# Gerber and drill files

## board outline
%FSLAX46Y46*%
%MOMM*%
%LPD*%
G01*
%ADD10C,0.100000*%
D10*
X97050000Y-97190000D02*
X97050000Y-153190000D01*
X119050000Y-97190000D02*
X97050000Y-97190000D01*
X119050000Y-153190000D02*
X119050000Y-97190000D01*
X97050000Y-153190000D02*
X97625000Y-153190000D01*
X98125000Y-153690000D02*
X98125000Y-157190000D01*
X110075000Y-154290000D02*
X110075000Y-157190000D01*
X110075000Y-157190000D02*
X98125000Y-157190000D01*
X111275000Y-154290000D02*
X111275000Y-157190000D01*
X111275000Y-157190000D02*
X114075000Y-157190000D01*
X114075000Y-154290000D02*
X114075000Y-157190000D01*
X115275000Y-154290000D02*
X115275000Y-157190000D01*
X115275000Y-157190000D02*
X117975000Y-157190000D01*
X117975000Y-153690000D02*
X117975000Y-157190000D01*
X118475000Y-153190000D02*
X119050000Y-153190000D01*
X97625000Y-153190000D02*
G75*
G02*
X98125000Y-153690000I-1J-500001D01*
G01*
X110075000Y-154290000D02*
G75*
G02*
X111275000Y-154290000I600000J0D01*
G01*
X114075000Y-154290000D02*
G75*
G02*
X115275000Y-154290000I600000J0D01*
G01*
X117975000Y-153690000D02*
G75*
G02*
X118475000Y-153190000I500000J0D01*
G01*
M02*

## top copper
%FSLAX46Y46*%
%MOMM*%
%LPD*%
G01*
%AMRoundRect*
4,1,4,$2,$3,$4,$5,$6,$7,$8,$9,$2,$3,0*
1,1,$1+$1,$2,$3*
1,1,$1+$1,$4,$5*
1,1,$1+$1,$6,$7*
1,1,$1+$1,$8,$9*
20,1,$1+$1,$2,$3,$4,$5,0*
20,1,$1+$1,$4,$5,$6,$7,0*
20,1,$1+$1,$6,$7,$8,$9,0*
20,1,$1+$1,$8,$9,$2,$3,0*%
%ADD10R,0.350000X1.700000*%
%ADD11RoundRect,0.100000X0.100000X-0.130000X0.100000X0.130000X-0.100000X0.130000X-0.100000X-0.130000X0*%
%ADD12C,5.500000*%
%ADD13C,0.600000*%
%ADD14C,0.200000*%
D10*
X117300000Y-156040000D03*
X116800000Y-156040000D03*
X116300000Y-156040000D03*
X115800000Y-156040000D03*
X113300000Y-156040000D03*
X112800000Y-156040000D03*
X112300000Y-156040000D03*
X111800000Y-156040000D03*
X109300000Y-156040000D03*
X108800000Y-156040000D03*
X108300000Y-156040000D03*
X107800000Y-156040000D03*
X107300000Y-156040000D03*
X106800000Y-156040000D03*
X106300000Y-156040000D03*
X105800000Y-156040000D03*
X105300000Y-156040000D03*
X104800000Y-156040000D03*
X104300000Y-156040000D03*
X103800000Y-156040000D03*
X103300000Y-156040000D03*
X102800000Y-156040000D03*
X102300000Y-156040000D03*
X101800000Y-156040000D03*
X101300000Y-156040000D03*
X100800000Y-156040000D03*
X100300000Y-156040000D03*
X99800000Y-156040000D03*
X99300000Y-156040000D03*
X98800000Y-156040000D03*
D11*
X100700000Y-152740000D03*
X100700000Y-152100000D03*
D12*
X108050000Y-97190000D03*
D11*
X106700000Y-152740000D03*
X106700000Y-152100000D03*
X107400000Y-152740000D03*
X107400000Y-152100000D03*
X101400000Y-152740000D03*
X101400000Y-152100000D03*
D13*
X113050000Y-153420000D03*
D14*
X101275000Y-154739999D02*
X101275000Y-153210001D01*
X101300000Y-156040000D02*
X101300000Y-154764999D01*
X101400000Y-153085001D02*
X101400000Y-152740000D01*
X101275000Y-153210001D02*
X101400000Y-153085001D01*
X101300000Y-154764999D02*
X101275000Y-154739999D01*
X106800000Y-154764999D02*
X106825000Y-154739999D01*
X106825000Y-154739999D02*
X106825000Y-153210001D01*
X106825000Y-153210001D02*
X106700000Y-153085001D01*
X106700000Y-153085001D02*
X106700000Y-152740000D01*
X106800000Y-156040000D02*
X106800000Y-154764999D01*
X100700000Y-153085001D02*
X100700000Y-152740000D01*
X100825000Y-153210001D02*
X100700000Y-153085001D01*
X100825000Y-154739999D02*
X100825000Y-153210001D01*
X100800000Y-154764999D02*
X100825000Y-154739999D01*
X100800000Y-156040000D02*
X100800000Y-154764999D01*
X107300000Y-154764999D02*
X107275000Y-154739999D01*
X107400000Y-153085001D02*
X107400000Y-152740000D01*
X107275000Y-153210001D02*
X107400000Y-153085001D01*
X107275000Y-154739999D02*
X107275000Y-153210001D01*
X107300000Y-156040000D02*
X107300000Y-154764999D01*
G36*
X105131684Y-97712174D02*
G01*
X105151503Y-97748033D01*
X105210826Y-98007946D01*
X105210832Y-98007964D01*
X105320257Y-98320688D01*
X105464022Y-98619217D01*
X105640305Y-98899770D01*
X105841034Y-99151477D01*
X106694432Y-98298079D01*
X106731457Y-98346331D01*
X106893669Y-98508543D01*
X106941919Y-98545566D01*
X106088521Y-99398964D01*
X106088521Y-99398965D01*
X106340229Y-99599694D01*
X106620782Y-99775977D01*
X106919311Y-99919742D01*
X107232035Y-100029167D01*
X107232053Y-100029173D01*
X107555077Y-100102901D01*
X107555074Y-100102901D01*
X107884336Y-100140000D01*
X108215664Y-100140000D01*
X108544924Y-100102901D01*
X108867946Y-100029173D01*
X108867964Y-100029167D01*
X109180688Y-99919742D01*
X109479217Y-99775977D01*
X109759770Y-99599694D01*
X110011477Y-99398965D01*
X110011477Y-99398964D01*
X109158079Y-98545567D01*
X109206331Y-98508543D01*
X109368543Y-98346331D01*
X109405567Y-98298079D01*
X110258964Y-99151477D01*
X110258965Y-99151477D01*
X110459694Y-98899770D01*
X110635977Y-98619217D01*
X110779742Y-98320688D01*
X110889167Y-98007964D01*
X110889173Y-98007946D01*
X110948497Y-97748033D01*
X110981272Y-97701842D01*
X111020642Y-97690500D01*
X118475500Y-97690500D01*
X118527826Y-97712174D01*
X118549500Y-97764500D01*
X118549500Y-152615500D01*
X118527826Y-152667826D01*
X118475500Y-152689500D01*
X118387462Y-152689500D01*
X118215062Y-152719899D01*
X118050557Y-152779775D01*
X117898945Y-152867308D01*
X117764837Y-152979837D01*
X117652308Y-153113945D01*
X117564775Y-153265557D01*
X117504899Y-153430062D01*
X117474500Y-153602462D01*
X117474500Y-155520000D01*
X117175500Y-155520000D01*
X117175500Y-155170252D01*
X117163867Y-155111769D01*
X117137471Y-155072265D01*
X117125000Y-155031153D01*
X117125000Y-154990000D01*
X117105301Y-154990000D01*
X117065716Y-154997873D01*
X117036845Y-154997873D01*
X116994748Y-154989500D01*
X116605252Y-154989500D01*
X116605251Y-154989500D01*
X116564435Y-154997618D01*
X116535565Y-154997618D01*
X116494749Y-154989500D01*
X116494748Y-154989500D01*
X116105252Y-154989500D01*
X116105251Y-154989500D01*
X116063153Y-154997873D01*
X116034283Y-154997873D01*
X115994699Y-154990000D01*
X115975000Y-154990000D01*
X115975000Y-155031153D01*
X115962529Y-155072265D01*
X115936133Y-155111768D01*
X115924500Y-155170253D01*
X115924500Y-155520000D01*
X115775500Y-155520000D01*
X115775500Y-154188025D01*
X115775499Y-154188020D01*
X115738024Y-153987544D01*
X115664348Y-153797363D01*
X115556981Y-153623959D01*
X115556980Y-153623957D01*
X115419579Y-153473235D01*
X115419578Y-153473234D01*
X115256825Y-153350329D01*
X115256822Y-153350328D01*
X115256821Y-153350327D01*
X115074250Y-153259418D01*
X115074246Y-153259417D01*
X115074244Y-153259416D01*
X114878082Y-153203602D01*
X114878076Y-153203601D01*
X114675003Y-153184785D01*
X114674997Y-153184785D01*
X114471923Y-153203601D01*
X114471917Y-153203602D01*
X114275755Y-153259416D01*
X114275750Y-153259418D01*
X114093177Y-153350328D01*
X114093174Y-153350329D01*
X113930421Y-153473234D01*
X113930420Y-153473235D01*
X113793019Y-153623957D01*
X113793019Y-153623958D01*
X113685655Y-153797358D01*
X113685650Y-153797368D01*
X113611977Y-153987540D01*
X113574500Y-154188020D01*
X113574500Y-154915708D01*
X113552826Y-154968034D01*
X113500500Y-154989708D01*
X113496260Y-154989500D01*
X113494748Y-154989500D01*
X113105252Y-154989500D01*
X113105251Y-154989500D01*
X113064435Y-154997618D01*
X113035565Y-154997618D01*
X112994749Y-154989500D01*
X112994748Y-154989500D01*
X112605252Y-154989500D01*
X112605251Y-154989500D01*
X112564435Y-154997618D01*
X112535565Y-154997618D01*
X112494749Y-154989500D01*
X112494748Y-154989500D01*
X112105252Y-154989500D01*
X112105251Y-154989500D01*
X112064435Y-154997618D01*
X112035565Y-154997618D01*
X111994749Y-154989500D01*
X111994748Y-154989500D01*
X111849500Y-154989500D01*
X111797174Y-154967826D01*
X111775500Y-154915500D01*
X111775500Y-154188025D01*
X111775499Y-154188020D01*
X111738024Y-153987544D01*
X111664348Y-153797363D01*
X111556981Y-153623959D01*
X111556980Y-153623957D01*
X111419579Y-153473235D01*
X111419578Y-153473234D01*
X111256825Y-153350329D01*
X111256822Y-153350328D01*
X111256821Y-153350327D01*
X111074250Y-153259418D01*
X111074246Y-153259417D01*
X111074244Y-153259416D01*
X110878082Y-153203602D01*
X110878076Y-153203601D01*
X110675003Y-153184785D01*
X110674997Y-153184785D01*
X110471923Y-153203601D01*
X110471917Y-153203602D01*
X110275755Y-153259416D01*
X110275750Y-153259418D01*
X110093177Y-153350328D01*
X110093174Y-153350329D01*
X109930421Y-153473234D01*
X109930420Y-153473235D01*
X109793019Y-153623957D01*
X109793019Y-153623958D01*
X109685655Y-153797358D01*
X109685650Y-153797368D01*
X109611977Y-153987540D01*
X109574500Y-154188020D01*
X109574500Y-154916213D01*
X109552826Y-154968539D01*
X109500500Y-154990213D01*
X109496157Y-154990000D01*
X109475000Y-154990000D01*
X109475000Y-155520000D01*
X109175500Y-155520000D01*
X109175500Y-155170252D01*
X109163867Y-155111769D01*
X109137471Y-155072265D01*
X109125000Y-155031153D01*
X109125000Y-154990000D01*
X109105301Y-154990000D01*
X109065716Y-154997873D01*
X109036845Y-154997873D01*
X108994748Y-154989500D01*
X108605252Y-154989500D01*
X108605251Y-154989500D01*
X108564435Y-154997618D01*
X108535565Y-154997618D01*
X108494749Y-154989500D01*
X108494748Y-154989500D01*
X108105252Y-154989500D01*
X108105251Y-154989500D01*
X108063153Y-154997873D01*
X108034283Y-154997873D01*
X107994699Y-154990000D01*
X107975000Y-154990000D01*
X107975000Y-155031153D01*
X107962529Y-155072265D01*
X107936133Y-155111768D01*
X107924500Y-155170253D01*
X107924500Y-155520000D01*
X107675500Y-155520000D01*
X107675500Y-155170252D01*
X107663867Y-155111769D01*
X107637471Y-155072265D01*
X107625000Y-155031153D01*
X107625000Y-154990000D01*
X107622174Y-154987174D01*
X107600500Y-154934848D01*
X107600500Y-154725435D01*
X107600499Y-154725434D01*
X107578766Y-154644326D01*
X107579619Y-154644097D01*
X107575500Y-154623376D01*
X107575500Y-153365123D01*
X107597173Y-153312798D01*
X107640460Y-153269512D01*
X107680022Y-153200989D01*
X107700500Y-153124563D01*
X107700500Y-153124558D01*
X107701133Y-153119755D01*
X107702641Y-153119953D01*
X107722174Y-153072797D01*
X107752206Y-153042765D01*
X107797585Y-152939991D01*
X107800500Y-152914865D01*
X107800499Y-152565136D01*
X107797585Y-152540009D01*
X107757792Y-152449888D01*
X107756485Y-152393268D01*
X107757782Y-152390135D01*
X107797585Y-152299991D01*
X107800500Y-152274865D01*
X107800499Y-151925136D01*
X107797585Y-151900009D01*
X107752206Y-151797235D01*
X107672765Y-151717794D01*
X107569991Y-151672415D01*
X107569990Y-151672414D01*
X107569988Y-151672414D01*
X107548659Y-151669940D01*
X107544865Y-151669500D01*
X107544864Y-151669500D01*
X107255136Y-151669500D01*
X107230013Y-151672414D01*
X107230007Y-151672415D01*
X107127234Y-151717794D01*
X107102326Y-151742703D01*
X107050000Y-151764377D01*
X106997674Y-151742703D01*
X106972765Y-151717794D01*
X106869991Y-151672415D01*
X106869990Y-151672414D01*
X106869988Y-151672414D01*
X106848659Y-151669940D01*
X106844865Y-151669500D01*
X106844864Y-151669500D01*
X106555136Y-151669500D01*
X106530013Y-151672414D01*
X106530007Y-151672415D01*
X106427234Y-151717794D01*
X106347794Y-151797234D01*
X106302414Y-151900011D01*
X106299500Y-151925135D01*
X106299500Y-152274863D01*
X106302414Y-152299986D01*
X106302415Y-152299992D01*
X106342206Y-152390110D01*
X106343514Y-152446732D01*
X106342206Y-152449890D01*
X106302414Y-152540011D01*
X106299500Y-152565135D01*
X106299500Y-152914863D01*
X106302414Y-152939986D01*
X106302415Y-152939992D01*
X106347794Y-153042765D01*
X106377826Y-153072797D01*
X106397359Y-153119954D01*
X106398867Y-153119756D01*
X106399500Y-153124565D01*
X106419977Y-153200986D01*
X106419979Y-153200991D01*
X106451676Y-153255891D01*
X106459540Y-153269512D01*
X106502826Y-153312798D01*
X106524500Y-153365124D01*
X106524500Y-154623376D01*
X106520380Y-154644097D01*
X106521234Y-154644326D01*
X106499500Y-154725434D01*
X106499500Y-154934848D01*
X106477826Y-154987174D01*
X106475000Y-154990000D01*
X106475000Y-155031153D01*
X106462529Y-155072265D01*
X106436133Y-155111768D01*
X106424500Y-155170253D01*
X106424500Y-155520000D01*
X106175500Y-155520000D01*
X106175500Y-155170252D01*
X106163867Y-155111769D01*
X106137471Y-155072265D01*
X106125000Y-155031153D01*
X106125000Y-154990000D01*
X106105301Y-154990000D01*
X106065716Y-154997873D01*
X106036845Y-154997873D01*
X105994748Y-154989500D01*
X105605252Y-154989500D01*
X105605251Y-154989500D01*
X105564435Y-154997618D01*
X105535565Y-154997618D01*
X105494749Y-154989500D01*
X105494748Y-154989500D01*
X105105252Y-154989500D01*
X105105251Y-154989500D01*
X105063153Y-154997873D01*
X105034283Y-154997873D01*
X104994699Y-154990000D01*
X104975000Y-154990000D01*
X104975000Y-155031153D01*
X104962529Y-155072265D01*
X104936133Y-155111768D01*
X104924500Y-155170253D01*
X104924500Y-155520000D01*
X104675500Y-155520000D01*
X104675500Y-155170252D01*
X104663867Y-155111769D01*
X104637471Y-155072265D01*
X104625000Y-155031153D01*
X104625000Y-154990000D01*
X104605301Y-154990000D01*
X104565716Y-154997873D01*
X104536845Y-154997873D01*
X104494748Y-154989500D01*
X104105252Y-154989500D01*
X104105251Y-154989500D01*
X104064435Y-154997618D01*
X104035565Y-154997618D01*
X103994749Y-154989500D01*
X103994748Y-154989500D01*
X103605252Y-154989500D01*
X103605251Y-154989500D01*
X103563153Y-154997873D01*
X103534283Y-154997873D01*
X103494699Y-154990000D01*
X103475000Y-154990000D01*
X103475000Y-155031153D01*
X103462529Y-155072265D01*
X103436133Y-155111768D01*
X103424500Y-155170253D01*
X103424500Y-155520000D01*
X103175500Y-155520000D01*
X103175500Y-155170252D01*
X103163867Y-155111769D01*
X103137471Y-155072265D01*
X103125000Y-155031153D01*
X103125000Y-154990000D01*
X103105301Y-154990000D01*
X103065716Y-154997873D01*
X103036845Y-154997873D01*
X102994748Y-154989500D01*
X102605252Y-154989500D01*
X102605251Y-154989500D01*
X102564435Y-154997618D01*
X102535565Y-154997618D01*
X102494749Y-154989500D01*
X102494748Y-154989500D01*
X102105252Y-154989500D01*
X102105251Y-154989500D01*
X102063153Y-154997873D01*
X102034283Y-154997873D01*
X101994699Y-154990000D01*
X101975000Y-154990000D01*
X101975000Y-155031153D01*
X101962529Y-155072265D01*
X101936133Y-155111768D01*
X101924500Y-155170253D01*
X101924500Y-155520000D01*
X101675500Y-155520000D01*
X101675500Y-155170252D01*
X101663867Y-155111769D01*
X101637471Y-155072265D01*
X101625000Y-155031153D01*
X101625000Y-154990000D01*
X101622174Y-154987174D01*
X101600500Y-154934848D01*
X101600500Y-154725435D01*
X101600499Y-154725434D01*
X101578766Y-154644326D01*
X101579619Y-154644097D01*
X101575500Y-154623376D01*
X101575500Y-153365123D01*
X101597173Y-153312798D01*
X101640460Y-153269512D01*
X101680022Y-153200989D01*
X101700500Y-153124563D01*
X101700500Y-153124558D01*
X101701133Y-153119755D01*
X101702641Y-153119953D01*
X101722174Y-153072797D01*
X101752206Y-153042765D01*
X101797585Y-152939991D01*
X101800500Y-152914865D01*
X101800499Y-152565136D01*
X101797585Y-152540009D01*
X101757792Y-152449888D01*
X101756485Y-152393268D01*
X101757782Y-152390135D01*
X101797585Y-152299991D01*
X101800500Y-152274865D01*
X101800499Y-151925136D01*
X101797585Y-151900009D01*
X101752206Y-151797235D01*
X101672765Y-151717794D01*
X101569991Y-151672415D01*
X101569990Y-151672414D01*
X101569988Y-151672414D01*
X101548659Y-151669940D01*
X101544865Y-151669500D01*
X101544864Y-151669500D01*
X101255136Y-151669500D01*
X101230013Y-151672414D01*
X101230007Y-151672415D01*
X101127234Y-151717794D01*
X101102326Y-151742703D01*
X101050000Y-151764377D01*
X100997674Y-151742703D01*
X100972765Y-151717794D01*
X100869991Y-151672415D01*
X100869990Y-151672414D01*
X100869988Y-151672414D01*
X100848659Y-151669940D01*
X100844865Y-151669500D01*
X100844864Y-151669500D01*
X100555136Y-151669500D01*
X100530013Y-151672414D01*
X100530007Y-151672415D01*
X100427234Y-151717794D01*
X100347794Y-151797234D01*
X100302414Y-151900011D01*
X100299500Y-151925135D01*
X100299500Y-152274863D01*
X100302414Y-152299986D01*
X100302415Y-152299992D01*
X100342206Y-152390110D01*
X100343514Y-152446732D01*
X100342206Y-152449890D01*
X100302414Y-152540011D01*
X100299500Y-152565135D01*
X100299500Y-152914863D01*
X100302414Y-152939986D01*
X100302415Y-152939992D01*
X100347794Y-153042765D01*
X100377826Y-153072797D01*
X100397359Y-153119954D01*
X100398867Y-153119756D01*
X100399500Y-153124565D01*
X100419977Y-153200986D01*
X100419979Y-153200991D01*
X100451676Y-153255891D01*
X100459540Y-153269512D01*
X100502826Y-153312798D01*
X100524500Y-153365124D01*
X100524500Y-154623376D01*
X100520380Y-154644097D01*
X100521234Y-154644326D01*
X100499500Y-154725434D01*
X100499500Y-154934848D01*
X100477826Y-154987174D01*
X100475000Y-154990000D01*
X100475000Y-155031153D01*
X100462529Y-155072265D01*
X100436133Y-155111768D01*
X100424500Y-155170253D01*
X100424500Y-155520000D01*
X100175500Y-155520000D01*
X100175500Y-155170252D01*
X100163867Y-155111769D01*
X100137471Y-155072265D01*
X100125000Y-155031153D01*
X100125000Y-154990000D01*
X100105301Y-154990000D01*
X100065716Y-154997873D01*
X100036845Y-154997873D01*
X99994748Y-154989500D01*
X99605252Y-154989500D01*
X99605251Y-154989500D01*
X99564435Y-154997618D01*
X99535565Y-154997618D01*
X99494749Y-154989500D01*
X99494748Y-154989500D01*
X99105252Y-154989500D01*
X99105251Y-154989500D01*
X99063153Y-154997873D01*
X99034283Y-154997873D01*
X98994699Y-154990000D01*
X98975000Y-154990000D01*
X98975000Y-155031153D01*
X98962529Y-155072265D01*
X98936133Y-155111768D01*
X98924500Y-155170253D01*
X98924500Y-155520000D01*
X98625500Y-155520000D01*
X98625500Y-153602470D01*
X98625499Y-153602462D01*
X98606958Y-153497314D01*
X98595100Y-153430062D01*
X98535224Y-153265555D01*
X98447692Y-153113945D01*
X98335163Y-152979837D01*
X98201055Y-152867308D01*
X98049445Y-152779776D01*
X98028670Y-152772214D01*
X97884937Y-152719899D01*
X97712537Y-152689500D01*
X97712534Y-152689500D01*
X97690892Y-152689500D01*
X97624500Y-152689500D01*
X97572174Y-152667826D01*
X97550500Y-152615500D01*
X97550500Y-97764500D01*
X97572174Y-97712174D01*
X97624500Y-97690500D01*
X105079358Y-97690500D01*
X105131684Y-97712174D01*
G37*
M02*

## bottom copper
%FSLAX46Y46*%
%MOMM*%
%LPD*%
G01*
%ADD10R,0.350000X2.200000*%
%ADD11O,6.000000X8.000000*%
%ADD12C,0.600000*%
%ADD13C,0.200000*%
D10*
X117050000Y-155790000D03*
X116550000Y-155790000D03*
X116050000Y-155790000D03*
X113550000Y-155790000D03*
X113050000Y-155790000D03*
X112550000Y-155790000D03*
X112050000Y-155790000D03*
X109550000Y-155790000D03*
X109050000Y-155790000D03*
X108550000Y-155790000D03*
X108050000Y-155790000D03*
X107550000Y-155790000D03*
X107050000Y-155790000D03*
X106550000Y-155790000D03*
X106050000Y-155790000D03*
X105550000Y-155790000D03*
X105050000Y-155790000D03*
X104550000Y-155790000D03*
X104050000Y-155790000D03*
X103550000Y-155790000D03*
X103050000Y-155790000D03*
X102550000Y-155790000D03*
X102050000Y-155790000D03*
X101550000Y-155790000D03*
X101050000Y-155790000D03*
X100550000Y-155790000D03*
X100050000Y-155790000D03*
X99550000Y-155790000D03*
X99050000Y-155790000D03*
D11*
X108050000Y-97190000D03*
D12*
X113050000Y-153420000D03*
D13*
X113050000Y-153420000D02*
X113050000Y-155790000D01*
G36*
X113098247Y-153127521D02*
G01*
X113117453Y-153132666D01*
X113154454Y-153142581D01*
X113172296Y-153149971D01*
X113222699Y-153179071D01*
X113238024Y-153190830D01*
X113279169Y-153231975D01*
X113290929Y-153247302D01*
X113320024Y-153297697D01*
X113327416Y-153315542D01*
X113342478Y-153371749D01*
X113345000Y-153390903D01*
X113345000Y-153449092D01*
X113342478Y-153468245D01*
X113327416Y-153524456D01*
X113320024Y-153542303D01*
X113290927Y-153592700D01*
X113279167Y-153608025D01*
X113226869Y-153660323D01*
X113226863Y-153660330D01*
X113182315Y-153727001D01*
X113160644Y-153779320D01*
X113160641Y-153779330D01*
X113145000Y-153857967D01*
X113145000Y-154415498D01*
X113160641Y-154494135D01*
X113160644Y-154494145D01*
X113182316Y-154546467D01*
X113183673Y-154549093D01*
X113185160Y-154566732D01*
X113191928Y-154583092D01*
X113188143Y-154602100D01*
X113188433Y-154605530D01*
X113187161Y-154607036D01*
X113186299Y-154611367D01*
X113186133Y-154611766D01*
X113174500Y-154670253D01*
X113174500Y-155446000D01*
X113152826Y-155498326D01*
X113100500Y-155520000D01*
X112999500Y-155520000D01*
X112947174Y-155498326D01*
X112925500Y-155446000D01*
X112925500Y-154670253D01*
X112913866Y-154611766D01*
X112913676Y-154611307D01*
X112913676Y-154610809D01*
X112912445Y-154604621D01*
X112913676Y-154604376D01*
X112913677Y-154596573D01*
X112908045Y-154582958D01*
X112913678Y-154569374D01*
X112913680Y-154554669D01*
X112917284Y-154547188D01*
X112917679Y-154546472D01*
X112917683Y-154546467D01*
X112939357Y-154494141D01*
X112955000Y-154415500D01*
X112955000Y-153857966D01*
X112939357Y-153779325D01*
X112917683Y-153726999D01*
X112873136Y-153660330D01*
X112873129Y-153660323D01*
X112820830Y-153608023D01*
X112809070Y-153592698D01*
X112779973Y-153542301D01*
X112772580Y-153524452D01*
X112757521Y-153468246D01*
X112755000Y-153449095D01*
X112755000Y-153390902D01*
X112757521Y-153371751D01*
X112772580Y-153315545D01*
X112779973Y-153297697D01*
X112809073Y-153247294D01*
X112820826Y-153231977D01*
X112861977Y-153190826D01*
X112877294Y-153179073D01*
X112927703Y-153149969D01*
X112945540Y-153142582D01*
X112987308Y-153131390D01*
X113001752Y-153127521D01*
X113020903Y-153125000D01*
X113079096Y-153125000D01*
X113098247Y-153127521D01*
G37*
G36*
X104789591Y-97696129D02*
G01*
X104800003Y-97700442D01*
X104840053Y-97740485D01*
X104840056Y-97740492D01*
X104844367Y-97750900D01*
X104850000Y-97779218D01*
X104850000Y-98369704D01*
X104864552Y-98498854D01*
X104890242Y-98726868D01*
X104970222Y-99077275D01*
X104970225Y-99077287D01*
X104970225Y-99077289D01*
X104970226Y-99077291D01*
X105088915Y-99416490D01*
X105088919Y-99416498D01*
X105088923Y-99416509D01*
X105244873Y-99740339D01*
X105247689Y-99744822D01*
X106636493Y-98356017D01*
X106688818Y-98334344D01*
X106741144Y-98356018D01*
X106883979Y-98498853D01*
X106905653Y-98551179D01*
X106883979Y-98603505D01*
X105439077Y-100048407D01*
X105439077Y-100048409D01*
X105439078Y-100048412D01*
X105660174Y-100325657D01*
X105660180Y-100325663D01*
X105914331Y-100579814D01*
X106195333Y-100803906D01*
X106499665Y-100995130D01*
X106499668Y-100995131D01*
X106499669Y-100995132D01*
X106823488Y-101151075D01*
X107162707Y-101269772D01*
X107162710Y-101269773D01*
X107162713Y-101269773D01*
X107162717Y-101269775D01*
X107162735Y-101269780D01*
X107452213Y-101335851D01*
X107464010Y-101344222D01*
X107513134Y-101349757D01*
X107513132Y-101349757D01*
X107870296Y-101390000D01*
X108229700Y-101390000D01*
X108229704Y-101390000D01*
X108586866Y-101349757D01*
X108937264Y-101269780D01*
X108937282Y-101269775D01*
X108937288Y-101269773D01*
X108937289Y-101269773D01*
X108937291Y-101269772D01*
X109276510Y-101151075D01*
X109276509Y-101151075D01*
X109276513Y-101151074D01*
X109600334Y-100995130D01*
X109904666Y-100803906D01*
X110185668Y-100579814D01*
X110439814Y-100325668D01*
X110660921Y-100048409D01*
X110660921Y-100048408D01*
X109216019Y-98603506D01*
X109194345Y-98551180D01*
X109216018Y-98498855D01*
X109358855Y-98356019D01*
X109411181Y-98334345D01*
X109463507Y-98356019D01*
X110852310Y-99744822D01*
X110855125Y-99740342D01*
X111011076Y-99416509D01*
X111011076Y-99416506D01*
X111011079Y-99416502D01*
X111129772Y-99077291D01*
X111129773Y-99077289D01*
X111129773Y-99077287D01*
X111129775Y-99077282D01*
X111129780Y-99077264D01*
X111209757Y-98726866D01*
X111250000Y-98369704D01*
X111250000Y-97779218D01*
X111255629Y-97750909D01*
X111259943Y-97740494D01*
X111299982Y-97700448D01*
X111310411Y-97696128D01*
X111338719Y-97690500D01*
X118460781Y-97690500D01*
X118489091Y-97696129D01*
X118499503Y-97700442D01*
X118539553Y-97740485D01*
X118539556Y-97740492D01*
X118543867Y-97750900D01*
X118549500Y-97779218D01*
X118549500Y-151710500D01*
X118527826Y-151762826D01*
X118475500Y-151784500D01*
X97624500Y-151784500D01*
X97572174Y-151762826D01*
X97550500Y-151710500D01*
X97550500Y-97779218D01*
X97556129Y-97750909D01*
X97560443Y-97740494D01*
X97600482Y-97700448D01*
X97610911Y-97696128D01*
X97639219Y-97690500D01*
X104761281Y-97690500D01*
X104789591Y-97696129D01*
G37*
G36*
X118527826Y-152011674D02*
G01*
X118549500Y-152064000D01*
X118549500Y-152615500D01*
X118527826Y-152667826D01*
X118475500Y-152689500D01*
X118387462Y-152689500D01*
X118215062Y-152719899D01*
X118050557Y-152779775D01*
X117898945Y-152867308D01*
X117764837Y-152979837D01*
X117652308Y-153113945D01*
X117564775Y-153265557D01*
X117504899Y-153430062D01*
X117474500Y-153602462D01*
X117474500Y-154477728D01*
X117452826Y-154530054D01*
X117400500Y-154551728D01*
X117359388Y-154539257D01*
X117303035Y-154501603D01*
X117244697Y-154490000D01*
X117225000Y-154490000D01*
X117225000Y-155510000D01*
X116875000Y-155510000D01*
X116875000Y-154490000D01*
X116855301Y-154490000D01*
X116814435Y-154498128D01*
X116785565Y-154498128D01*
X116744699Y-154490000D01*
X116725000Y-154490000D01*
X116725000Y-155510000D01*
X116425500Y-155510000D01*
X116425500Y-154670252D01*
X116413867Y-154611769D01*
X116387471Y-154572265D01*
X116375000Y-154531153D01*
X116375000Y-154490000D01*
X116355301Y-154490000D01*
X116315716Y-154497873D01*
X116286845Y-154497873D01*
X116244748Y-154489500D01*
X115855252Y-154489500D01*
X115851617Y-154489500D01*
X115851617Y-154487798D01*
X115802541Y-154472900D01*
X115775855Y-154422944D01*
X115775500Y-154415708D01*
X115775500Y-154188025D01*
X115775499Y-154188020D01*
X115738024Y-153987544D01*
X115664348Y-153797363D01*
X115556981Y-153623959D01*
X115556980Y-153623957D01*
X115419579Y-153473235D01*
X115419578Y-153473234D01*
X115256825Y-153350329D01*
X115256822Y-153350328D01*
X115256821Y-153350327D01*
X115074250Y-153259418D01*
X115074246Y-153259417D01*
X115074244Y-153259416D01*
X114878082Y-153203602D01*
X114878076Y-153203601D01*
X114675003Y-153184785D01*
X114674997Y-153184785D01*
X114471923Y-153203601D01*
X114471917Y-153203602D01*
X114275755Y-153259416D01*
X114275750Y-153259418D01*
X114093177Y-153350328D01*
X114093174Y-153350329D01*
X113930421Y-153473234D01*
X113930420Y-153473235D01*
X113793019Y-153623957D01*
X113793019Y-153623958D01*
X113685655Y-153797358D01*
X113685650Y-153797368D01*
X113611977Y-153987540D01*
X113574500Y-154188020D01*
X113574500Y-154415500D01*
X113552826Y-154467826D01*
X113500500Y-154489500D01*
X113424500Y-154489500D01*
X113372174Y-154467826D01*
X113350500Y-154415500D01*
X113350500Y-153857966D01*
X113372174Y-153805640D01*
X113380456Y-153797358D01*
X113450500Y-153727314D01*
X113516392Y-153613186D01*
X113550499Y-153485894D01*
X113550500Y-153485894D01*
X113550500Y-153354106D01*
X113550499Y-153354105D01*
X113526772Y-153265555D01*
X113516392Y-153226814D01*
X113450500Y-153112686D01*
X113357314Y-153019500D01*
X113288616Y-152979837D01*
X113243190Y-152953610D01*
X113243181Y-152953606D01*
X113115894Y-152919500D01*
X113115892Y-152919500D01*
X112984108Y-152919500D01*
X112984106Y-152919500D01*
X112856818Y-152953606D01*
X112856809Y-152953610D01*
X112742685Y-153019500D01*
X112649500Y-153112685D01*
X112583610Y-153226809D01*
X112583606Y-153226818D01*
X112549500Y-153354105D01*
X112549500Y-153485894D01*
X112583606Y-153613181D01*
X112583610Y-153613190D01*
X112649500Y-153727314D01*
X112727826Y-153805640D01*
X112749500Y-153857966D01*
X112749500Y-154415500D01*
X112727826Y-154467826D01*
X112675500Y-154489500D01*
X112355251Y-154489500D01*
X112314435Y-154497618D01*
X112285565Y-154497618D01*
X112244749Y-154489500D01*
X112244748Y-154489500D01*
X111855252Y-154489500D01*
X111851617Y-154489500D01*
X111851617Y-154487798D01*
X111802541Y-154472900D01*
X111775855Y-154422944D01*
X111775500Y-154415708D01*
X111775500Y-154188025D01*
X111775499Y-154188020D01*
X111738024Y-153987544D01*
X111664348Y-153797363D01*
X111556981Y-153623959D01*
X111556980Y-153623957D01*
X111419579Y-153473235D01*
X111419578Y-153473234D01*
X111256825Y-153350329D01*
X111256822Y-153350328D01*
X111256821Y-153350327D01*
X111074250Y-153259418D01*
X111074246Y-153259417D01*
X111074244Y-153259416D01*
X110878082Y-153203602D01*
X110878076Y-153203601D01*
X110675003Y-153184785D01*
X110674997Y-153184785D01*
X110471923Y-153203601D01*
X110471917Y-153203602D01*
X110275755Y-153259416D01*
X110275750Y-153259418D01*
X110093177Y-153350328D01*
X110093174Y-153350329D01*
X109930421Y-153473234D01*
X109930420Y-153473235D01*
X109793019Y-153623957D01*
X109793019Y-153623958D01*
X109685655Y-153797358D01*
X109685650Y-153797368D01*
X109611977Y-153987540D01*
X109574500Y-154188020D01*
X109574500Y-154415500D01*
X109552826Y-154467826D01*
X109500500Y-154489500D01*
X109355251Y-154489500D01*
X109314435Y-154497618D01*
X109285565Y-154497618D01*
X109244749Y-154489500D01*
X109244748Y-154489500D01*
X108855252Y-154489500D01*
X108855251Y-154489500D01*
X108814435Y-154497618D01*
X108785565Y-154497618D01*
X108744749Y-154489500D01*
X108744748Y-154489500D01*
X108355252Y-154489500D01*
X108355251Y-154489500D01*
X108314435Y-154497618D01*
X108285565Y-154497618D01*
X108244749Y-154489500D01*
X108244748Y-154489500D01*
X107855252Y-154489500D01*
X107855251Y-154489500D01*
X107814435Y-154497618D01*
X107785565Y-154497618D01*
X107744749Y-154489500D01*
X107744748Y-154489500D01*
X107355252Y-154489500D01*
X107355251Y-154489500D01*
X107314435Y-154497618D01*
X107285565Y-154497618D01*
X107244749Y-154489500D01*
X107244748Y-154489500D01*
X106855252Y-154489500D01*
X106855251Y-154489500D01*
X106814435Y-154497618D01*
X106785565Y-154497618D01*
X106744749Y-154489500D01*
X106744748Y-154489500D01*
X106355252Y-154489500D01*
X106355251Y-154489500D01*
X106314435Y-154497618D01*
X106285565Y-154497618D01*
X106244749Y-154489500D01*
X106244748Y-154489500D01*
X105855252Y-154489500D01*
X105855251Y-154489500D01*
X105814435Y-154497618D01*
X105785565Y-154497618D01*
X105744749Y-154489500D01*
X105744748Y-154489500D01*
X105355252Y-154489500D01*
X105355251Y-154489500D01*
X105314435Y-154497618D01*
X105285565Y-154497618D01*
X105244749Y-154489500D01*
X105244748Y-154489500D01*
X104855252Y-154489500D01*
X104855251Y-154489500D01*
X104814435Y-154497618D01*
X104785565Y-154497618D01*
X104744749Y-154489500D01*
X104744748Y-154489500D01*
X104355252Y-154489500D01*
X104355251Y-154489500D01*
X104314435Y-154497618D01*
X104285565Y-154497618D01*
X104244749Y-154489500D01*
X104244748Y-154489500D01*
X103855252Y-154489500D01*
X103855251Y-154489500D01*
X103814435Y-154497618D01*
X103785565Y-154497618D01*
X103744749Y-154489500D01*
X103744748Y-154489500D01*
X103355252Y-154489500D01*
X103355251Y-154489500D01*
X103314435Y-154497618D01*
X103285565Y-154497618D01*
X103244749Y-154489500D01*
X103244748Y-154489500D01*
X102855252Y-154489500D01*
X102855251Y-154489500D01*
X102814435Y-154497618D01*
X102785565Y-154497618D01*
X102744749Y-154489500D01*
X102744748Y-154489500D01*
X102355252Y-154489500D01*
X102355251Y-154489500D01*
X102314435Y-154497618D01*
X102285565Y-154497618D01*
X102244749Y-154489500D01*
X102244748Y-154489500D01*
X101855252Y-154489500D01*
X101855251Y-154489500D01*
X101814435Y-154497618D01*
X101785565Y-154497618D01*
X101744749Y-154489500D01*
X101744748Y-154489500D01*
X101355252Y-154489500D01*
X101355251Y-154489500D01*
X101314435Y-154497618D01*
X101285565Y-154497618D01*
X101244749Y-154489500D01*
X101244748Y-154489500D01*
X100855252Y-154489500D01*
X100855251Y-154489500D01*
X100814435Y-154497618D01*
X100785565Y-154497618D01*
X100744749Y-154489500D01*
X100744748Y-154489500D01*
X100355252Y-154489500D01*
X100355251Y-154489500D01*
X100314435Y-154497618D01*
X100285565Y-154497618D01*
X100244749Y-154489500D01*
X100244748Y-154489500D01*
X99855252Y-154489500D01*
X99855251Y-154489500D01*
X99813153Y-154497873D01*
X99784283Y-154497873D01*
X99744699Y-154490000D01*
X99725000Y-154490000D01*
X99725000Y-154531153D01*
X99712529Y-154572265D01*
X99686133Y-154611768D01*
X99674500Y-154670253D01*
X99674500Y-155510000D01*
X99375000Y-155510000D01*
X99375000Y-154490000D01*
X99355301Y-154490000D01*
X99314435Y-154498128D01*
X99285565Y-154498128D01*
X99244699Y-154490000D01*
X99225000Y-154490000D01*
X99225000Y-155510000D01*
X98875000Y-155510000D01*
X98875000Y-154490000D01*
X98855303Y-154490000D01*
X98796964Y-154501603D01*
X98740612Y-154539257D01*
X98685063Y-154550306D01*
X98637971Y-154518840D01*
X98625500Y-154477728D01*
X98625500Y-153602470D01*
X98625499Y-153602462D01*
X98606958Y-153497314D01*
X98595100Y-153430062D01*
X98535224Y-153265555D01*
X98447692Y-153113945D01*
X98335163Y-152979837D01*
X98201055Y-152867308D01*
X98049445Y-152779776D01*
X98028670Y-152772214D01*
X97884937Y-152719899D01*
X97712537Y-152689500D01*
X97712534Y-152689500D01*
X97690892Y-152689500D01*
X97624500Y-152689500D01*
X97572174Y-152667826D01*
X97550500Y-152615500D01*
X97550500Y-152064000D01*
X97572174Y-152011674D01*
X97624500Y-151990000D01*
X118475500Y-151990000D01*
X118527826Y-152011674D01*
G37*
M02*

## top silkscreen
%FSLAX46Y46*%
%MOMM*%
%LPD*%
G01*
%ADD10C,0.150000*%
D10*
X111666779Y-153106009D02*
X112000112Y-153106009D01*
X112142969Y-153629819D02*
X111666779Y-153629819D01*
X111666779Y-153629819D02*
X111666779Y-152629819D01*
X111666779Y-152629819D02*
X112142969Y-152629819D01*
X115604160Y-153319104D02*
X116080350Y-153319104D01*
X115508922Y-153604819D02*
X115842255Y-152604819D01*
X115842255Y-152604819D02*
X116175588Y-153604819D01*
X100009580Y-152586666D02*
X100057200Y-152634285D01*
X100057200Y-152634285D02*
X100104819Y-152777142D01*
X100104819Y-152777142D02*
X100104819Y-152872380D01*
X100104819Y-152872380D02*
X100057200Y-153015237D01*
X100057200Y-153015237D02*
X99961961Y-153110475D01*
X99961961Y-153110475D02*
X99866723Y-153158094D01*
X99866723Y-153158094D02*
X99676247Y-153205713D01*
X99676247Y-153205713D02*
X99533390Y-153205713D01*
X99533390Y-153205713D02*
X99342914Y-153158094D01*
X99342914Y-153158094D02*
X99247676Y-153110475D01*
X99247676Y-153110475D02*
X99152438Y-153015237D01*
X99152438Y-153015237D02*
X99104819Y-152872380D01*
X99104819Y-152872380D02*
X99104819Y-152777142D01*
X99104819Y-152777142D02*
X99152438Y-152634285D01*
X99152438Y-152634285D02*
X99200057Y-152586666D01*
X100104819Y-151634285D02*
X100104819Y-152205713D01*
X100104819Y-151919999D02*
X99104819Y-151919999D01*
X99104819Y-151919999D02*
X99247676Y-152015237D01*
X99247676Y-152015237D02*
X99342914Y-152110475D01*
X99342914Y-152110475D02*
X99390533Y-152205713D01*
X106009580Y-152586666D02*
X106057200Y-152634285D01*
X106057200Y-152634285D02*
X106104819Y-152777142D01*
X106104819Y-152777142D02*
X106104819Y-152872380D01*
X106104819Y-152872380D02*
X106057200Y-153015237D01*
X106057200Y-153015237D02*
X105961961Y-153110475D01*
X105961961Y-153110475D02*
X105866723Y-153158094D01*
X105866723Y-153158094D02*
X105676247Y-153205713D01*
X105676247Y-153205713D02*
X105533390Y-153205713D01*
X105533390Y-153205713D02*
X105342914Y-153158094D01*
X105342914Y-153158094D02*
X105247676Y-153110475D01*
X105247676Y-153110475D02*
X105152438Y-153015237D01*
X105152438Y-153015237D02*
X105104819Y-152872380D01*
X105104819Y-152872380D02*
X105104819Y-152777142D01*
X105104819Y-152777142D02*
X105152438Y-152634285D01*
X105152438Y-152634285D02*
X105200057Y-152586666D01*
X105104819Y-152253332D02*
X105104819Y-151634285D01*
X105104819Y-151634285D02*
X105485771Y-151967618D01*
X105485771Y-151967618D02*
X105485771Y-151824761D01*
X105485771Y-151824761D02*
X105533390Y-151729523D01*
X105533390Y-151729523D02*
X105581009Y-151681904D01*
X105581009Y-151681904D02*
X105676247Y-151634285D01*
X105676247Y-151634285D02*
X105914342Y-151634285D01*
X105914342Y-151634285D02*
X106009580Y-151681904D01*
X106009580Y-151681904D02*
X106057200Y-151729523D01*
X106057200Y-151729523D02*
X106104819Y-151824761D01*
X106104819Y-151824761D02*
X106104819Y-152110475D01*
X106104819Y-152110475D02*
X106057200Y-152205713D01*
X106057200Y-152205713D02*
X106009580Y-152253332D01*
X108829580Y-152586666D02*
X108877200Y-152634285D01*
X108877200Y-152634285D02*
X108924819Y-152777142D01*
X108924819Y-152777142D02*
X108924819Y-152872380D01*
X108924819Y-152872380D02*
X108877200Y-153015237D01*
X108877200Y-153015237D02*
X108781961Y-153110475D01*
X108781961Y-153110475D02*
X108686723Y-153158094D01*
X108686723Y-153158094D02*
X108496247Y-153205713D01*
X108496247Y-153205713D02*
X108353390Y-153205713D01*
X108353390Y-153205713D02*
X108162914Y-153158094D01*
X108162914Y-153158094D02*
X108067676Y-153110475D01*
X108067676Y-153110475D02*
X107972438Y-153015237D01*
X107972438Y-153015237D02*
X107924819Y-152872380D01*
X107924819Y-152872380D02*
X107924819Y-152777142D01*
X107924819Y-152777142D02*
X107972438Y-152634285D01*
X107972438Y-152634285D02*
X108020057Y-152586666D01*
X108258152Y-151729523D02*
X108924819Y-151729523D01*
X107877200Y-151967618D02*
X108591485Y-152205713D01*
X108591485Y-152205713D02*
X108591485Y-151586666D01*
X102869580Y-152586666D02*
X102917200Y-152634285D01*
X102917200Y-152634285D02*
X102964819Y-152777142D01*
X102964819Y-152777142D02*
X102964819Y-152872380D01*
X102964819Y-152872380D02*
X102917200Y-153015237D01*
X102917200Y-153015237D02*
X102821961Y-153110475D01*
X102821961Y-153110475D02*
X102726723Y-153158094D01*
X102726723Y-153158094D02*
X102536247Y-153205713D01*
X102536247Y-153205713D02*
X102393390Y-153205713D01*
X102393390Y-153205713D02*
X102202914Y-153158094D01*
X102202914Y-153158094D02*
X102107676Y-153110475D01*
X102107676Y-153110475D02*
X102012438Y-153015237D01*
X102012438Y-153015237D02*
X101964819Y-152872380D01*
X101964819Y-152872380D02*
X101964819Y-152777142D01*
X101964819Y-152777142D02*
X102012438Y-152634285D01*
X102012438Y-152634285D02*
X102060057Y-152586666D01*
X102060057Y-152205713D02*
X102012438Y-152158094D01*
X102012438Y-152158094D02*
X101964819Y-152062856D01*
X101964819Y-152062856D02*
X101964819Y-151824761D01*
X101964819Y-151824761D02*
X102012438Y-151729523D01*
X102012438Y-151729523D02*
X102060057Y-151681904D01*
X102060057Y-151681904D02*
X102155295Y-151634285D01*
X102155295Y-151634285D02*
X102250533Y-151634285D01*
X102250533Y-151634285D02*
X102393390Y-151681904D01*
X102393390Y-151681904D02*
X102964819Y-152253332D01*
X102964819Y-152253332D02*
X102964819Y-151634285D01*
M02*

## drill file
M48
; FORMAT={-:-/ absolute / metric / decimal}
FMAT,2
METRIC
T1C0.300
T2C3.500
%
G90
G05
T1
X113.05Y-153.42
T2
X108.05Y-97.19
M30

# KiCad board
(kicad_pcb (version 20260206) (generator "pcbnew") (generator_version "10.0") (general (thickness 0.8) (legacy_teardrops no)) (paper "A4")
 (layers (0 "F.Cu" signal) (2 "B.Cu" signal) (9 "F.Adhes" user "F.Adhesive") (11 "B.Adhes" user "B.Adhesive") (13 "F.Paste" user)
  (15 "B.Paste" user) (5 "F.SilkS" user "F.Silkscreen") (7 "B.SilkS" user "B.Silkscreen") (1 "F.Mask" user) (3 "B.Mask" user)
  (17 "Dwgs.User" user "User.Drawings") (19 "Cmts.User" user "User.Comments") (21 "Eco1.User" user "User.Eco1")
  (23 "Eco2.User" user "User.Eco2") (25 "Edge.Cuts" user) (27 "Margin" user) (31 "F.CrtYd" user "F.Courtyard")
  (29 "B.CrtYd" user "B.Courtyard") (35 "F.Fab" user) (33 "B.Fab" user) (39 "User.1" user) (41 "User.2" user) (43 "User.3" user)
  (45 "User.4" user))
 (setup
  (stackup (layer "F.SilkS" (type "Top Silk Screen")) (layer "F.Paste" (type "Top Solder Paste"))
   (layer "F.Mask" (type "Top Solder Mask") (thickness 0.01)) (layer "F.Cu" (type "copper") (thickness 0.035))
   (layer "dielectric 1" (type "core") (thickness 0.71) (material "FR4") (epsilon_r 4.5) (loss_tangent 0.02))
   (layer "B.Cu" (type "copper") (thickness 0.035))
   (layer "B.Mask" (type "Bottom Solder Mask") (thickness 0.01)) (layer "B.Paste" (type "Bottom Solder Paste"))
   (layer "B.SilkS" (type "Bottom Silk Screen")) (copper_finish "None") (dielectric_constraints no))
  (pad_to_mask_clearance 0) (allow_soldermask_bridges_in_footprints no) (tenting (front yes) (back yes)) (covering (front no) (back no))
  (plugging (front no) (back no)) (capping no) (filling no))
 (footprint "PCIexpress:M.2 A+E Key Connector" (layer "F.Cu") (at 108.05 156.08)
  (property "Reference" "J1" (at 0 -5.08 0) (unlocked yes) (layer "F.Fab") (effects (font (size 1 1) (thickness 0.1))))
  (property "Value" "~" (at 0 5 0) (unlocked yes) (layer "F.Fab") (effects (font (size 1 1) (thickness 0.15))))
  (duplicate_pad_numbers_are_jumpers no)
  (fp_line (start -11 -2.89) (end -10.425 -2.89) (stroke (width 0.1) (type default)) (layer "Edge.Cuts"))
  (fp_line (start -9.925 -2.39) (end -9.925 1.11) (stroke (width 0.1) (type default)) (layer "Edge.Cuts"))
  (fp_line (start 2.025 -1.79) (end 2.025 1.11) (stroke (width 0.1) (type default)) (layer "Edge.Cuts"))
  (fp_line (start 2.025 1.11) (end -9.925 1.11) (stroke (width 0.1) (type default)) (layer "Edge.Cuts"))
  (fp_line (start 3.225 -1.79) (end 3.225 1.11) (stroke (width 0.1) (type default)) (layer "Edge.Cuts"))
  (fp_line (start 3.225 1.11) (end 6.025 1.11) (stroke (width 0.1) (type default)) (layer "Edge.Cuts"))
  (fp_line (start 6.025 -1.79) (end 6.025 1.11) (stroke (width 0.1) (type default)) (layer "Edge.Cuts"))
  (fp_line (start 7.225 -1.79) (end 7.225 1.11) (stroke (width 0.1) (type default)) (layer "Edge.Cuts"))
  (fp_line (start 7.225 1.11) (end 9.925 1.11) (stroke (width 0.1) (type default)) (layer "Edge.Cuts"))
  (fp_line (start 9.925 -2.39) (end 9.925 1.11) (stroke (width 0.1) (type default)) (layer "Edge.Cuts"))
  (fp_line (start 10.425 -2.89) (end 11 -2.89) (stroke (width 0.1) (type default)) (layer "Edge.Cuts"))
  (fp_arc (start -10.425 -2.89) (mid -10.071447 -2.743553) (end -9.925 -2.39) (stroke (width 0.1) (type default)) (layer "Edge.Cuts"))
  (fp_arc (start 2.025 -1.79) (mid 2.625 -2.39) (end 3.225 -1.79) (stroke (width 0.1) (type default)) (layer "Edge.Cuts"))
  (fp_arc (start 6.025 -1.79) (mid 6.625 -2.39) (end 7.225 -1.79) (stroke (width 0.1) (type default)) (layer "Edge.Cuts"))
  (fp_arc (start 9.925 -2.39) (mid 10.071447 -2.743553) (end 10.425 -2.89) (stroke (width 0.1) (type default)) (layer "Edge.Cuts"))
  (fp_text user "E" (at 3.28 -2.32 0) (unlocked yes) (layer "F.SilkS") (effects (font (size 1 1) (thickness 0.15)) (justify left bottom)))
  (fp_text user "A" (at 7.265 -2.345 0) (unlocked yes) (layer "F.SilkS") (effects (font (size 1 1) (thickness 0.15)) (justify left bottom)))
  (pad "1" smd rect (at 9.25 -0.04 180) (size 0.35 1.7) (layers "F.Cu") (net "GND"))
  (pad "2" smd rect (at 9 -0.29 180) (size 0.35 2.2) (layers "B.Cu") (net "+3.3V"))
  (pad "3" smd rect (at 8.75 -0.04 180) (size 0.35 1.7) (layers "F.Cu") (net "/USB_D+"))
  (pad "4" smd rect (at 8.5 -0.29 180) (size 0.35 2.2) (layers "B.Cu") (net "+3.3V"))
  (pad "5" smd rect (at 8.25 -0.04 180) (size 0.35 1.7) (layers "F.Cu") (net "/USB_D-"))
  (pad "6" smd rect (at 8 -0.29 180) (size 0.35 2.2) (layers "B.Cu") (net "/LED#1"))
  (pad "7" smd rect (at 7.75 -0.04 180) (size 0.35 1.7) (layers "F.Cu") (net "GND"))
  (pad "16" smd rect (at 5.5 -0.29 180) (size 0.35 2.2) (layers "B.Cu") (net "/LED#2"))
  (pad "17" smd rect (at 5.25 -0.04 180) (size 0.35 1.7) (layers "F.Cu") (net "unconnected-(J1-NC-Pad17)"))
  (pad "18" smd rect (at 5 -0.29 180) (size 0.35 2.2) (layers "B.Cu") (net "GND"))
  (pad "19" smd rect (at 4.75 -0.04 180) (size 0.35 1.7) (layers "F.Cu") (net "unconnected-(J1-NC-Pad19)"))
  (pad "20" smd rect (at 4.5 -0.29 180) (size 0.35 2.2) (layers "B.Cu") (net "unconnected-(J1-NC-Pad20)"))
  (pad "21" smd rect (at 4.25 -0.04 180) (size 0.35 1.7) (layers "F.Cu") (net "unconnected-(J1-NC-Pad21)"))
  (pad "22" smd rect (at 4 -0.29 180) (size 0.35 2.2) (layers "B.Cu") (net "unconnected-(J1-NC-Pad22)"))
  (pad "23" smd rect (at 3.75 -0.04 180) (size 0.35 1.7) (layers "F.Cu") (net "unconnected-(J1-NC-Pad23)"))
  (pad "32" smd rect (at 1.5 -0.29 180) (size 0.35 2.2) (layers "B.Cu") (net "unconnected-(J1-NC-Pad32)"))
  (pad "33" smd rect (at 1.25 -0.04 180) (size 0.35 1.7) (layers "F.Cu") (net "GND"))
  (pad "34" smd rect (at 1 -0.29 180) (size 0.35 2.2) (layers "B.Cu") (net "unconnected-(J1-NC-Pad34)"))
  (pad "35" smd rect (at 0.75 -0.04 180) (size 0.35 1.7) (layers "F.Cu") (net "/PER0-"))
  (pad "36" smd rect (at 0.5 -0.29 180) (size 0.35 2.2) (layers "B.Cu") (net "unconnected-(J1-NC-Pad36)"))
  (pad "37" smd rect (at 0.25 -0.04 180) (size 0.35 1.7) (layers "F.Cu") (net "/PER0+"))
  (pad "38" smd rect (at 0 -0.29 180) (size 0.35 2.2) (layers "B.Cu") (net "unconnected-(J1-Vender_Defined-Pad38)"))
  (pad "39" smd rect (at -0.25 -0.04 180) (size 0.35 1.7) (layers "F.Cu") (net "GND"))
  (pad "40" smd rect (at -0.5 -0.29 180) (size 0.35 2.2) (layers "B.Cu") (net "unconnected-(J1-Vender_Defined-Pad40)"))
  (pad "41" smd rect (at -0.75 -0.04 180) (size 0.35 1.7) (layers "F.Cu") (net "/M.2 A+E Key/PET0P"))
  (pad "42" smd rect (at -1 -0.29 180) (size 0.35 2.2) (layers "B.Cu") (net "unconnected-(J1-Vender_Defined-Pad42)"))
  (pad "43" smd rect (at -1.25 -0.04 180) (size 0.35 1.7) (layers "F.Cu") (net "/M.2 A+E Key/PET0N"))
  (pad "44" smd rect (at -1.5 -0.29 180) (size 0.35 2.2) (layers "B.Cu") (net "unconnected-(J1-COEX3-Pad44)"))
  (pad "45" smd rect (at -1.75 -0.04 180) (size 0.35 1.7) (layers "F.Cu") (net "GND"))
  (pad "46" smd rect (at -2 -0.29 180) (size 0.35 2.2) (layers "B.Cu") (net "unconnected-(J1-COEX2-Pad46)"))
  (pad "47" smd rect (at -2.25 -0.04 180) (size 0.35 1.7) (layers "F.Cu") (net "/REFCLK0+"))
  (pad "48" smd rect (at -2.5 -0.29 180) (size 0.35 2.2) (layers "B.Cu") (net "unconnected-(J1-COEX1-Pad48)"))
  (pad "49" smd rect (at -2.75 -0.04 180) (size 0.35 1.7) (layers "F.Cu") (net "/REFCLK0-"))
  (pad "50" smd rect (at -3 -0.29 180) (size 0.35 2.2) (layers "B.Cu") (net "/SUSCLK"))
  (pad "51" smd rect (at -3.25 -0.04 180) (size 0.35 1.7) (layers "F.Cu") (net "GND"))
  (pad "52" smd rect (at -3.5 -0.29 180) (size 0.35 2.2) (layers "B.Cu") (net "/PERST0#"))
  (pad "53" smd rect (at -3.75 -0.04 180) (size 0.35 1.7) (layers "F.Cu") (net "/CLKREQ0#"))
  (pad "54" smd rect (at -4 -0.29 180) (size 0.35 2.2) (layers "B.Cu") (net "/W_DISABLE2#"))
  (pad "55" smd rect (at -4.25 -0.04 180) (size 0.35 1.7) (layers "F.Cu") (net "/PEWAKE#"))
  (pad "56" smd rect (at -4.5 -0.29 180) (size 0.35 2.2) (layers "B.Cu") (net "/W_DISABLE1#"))
  (pad "57" smd rect (at -4.75 -0.04 180) (size 0.35 1.7) (layers "F.Cu") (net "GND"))
  (pad "58" smd rect (at -5 -0.29 180) (size 0.35 2.2) (layers "B.Cu") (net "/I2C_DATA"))
  (pad "59" smd rect (at -5.25 -0.04 180) (size 0.35 1.7) (layers "F.Cu") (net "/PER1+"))
  (pad "60" smd rect (at -5.5 -0.29 180) (size 0.35 2.2) (layers "B.Cu") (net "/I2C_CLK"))
  (pad "61" smd rect (at -5.75 -0.04 180) (size 0.35 1.7) (layers "F.Cu") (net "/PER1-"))
  (pad "62" smd rect (at -6 -0.29 180) (size 0.35 2.2) (layers "B.Cu") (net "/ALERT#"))
  (pad "63" smd rect (at -6.25 -0.04 180) (size 0.35 1.7) (layers "F.Cu") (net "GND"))
  (pad "64" smd rect (at -6.5 -0.29 180) (size 0.35 2.2) (layers "B.Cu") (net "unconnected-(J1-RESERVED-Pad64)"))
  (pad "65" smd rect (at -6.75 -0.04 180) (size 0.35 1.7) (layers "F.Cu") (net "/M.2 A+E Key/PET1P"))
  (pad "66" smd rect (at -7 -0.29 180) (size 0.35 2.2) (layers "B.Cu") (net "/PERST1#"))
  (pad "67" smd rect (at -7.25 -0.04 180) (size 0.35 1.7) (layers "F.Cu") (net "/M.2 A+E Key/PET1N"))
  (pad "68" smd rect (at -7.5 -0.29 180) (size 0.35 2.2) (layers "B.Cu") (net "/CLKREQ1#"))
  (pad "69" smd rect (at -7.75 -0.04 180) (size 0.35 1.7) (layers "F.Cu") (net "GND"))
  (pad "70" smd rect (at -8 -0.29 180) (size 0.35 2.2) (layers "B.Cu") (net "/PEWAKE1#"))
  (pad "71" smd rect (at -8.25 -0.04 180) (size 0.35 1.7) (layers "F.Cu") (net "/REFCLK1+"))
  (pad "72" smd rect (at -8.5 -0.29 180) (size 0.35 2.2) (layers "B.Cu") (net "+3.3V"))
  (pad "73" smd rect (at -8.75 -0.04 180) (size 0.35 1.7) (layers "F.Cu") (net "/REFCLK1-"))
  (pad "74" smd rect (at -9 -0.29 180) (size 0.35 2.2) (layers "B.Cu") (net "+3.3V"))
  (pad "75" smd rect (at -9.25 -0.04 180) (size 0.35 1.7) (layers "F.Cu") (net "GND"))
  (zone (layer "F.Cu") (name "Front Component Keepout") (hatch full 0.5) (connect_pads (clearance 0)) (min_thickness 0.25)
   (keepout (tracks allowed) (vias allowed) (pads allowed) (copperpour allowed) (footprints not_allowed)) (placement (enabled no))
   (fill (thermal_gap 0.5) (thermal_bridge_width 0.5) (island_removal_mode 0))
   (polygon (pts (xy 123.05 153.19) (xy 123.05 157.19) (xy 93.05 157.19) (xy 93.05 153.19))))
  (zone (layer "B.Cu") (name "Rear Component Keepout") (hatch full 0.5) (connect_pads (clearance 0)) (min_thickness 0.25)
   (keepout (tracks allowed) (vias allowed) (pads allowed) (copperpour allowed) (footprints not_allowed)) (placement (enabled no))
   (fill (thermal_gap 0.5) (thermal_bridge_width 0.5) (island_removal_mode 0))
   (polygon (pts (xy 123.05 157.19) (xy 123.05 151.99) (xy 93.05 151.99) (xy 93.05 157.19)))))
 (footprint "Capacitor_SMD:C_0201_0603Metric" (layer "F.Cu") (at 100.7 152.42 90)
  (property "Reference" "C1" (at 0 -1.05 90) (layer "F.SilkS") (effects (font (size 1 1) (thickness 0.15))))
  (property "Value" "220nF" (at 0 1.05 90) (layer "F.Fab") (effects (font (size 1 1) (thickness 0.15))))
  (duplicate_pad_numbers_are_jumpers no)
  (pad "" smd roundrect (at -0.345 0 90) (size 0.318 0.36) (layers "F.Paste") (roundrect_rratio 0.25))
  (pad "" smd roundrect (at 0.345 0 90) (size 0.318 0.36) (layers "F.Paste") (roundrect_rratio 0.25))
  (pad "1" smd roundrect (at -0.32 0 90) (size 0.46 0.4) (layers "F.Cu" "F.Mask") (roundrect_rratio 0.25) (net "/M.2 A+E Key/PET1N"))
  (pad "2" smd roundrect (at 0.32 0 90) (size 0.46 0.4) (layers "F.Cu" "F.Mask") (roundrect_rratio 0.25) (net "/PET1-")))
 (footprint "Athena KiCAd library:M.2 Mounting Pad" (layer "F.Cu") (at 108.05 97.19)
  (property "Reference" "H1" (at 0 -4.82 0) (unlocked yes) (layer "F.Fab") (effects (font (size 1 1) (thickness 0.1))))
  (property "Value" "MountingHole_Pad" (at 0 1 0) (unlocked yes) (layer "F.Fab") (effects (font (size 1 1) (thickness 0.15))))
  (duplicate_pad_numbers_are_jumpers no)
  (pad "1" thru_hole circle (at 0 0) (size 5.5 5.5) (drill 3.5) (layers "*.Cu" "*.Mask") (remove_unused_layers no) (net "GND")
   (padstack (mode front_inner_back)
    (layer "Inner" (shape circle) (size 5.5 5.5) (zone_connect -1)) (layer "B.Cu" (shape oval) (size 6 8) (zone_connect -1)))))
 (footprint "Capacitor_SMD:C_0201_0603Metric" (layer "F.Cu") (at 106.7 152.42 90)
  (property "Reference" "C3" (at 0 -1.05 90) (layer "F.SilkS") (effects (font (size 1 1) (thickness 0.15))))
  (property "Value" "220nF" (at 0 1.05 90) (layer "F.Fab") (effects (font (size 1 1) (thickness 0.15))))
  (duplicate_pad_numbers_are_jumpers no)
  (pad "" smd roundrect (at -0.345 0 90) (size 0.318 0.36) (layers "F.Paste") (roundrect_rratio 0.25))
  (pad "" smd roundrect (at 0.345 0 90) (size 0.318 0.36) (layers "F.Paste") (roundrect_rratio 0.25))
  (pad "1" smd roundrect (at -0.32 0 90) (size 0.46 0.4) (layers "F.Cu" "F.Mask") (roundrect_rratio 0.25) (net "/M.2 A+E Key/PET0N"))
  (pad "2" smd roundrect (at 0.32 0 90) (size 0.46 0.4) (layers "F.Cu" "F.Mask") (roundrect_rratio 0.25) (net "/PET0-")))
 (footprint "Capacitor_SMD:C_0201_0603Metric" (layer "F.Cu") (at 107.4 152.42 90)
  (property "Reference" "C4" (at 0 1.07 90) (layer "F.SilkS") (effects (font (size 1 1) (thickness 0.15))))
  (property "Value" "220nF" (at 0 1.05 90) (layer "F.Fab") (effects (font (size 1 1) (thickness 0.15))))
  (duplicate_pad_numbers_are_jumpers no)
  (pad "" smd roundrect (at -0.345 0 90) (size 0.318 0.36) (layers "F.Paste") (roundrect_rratio 0.25))
  (pad "" smd roundrect (at 0.345 0 90) (size 0.318 0.36) (layers "F.Paste") (roundrect_rratio 0.25))
  (pad "1" smd roundrect (at -0.32 0 90) (size 0.46 0.4) (layers "F.Cu" "F.Mask") (roundrect_rratio 0.25) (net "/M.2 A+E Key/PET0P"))
  (pad "2" smd roundrect (at 0.32 0 90) (size 0.46 0.4) (layers "F.Cu" "F.Mask") (roundrect_rratio 0.25) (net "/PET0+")))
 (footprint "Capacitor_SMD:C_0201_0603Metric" (layer "F.Cu") (at 101.4 152.42 90)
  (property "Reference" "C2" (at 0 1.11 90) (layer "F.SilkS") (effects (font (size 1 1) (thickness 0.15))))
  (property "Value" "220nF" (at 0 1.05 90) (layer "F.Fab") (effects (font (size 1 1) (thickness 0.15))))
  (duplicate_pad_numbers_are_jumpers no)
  (pad "" smd roundrect (at -0.345 0 90) (size 0.318 0.36) (layers "F.Paste") (roundrect_rratio 0.25))
  (pad "" smd roundrect (at 0.345 0 90) (size 0.318 0.36) (layers "F.Paste") (roundrect_rratio 0.25))
  (pad "1" smd roundrect (at -0.32 0 90) (size 0.46 0.4) (layers "F.Cu" "F.Mask") (roundrect_rratio 0.25) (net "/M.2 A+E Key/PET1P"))
  (pad "2" smd roundrect (at 0.32 0 90) (size 0.46 0.4) (layers "F.Cu" "F.Mask") (roundrect_rratio 0.25) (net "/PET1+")))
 (gr_line (start 97.05 97.19) (end 97.05 153.19) (stroke (width 0.1) (type default)) (layer "Edge.Cuts"))
 (gr_line (start 119.05 97.19) (end 97.05 97.19) (stroke (width 0.1) (type default)) (layer "Edge.Cuts"))
 (gr_line (start 119.05 153.19) (end 119.05 97.19) (stroke (width 0.1) (type default)) (layer "Edge.Cuts"))
 (via (at 113.05 153.42) (size 0.6) (drill 0.3) (layers "F.Cu" "B.Cu") (free yes) (capping no) (covering (front no) (back no))
  (plugging (front no) (back no)) (filling no) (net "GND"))
 (segment (start 113.05 153.42) (end 113.05 155.79) (width 0.2) (layer "B.Cu") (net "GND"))
 (segment (start 101.275 154.739999) (end 101.275 153.210001) (width 0.2) (layer "F.Cu") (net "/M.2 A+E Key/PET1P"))
 (segment (start 101.3 156.04) (end 101.3 154.764999) (width 0.2) (layer "F.Cu") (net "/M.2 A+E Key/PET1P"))
 (segment (start 101.4 153.085001) (end 101.4 152.74) (width 0.2) (layer "F.Cu") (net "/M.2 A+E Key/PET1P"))
 (segment (start 101.275 153.210001) (end 101.4 153.085001) (width 0.2) (layer "F.Cu") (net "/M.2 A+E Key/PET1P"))
 (segment (start 101.3 154.764999) (end 101.275 154.739999) (width 0.2) (layer "F.Cu") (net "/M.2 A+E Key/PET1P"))
 (segment (start 106.8 154.764999) (end 106.825 154.739999) (width 0.2) (layer "F.Cu") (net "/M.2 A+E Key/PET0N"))
 (segment (start 106.825 154.739999) (end 106.825 153.210001) (width 0.2) (layer "F.Cu") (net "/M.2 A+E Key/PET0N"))
 (segment (start 106.825 153.210001) (end 106.7 153.085001) (width 0.2) (layer "F.Cu") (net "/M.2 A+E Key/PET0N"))
 (segment (start 106.7 153.085001) (end 106.7 152.74) (width 0.2) (layer "F.Cu") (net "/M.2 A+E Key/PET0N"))
 (segment (start 106.8 156.04) (end 106.8 154.764999) (width 0.2) (layer "F.Cu") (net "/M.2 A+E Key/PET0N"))
 (segment (start 100.7 153.085001) (end 100.7 152.74) (width 0.2) (layer "F.Cu") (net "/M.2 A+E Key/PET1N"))
 (segment (start 100.825 153.210001) (end 100.7 153.085001) (width 0.2) (layer "F.Cu") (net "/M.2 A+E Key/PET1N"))
 (segment (start 100.825 154.739999) (end 100.825 153.210001) (width 0.2) (layer "F.Cu") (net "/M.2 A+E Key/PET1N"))
 (segment (start 100.8 154.764999) (end 100.825 154.739999) (width 0.2) (layer "F.Cu") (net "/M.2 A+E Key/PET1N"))
 (segment (start 100.8 156.04) (end 100.8 154.764999) (width 0.2) (layer "F.Cu") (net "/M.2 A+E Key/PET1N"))
 (segment (start 107.3 154.764999) (end 107.275 154.739999) (width 0.2) (layer "F.Cu") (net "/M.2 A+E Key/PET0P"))
 (segment (start 107.4 153.085001) (end 107.4 152.74) (width 0.2) (layer "F.Cu") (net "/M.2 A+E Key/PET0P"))
 (segment (start 107.275 153.210001) (end 107.4 153.085001) (width 0.2) (layer "F.Cu") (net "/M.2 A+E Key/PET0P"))
 (segment (start 107.275 154.739999) (end 107.275 153.210001) (width 0.2) (layer "F.Cu") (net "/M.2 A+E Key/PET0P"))
 (segment (start 107.3 156.04) (end 107.3 154.764999) (width 0.2) (layer "F.Cu") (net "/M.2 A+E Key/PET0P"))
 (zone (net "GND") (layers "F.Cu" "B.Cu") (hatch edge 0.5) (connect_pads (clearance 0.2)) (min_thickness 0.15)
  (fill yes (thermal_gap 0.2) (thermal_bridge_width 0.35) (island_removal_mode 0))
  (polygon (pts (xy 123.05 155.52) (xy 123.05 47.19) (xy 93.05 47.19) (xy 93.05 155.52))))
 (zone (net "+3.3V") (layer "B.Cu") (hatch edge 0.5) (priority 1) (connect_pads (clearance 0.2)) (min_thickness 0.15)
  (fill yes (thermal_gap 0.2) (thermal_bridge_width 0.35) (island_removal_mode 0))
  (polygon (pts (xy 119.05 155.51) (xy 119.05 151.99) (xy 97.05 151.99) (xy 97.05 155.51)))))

